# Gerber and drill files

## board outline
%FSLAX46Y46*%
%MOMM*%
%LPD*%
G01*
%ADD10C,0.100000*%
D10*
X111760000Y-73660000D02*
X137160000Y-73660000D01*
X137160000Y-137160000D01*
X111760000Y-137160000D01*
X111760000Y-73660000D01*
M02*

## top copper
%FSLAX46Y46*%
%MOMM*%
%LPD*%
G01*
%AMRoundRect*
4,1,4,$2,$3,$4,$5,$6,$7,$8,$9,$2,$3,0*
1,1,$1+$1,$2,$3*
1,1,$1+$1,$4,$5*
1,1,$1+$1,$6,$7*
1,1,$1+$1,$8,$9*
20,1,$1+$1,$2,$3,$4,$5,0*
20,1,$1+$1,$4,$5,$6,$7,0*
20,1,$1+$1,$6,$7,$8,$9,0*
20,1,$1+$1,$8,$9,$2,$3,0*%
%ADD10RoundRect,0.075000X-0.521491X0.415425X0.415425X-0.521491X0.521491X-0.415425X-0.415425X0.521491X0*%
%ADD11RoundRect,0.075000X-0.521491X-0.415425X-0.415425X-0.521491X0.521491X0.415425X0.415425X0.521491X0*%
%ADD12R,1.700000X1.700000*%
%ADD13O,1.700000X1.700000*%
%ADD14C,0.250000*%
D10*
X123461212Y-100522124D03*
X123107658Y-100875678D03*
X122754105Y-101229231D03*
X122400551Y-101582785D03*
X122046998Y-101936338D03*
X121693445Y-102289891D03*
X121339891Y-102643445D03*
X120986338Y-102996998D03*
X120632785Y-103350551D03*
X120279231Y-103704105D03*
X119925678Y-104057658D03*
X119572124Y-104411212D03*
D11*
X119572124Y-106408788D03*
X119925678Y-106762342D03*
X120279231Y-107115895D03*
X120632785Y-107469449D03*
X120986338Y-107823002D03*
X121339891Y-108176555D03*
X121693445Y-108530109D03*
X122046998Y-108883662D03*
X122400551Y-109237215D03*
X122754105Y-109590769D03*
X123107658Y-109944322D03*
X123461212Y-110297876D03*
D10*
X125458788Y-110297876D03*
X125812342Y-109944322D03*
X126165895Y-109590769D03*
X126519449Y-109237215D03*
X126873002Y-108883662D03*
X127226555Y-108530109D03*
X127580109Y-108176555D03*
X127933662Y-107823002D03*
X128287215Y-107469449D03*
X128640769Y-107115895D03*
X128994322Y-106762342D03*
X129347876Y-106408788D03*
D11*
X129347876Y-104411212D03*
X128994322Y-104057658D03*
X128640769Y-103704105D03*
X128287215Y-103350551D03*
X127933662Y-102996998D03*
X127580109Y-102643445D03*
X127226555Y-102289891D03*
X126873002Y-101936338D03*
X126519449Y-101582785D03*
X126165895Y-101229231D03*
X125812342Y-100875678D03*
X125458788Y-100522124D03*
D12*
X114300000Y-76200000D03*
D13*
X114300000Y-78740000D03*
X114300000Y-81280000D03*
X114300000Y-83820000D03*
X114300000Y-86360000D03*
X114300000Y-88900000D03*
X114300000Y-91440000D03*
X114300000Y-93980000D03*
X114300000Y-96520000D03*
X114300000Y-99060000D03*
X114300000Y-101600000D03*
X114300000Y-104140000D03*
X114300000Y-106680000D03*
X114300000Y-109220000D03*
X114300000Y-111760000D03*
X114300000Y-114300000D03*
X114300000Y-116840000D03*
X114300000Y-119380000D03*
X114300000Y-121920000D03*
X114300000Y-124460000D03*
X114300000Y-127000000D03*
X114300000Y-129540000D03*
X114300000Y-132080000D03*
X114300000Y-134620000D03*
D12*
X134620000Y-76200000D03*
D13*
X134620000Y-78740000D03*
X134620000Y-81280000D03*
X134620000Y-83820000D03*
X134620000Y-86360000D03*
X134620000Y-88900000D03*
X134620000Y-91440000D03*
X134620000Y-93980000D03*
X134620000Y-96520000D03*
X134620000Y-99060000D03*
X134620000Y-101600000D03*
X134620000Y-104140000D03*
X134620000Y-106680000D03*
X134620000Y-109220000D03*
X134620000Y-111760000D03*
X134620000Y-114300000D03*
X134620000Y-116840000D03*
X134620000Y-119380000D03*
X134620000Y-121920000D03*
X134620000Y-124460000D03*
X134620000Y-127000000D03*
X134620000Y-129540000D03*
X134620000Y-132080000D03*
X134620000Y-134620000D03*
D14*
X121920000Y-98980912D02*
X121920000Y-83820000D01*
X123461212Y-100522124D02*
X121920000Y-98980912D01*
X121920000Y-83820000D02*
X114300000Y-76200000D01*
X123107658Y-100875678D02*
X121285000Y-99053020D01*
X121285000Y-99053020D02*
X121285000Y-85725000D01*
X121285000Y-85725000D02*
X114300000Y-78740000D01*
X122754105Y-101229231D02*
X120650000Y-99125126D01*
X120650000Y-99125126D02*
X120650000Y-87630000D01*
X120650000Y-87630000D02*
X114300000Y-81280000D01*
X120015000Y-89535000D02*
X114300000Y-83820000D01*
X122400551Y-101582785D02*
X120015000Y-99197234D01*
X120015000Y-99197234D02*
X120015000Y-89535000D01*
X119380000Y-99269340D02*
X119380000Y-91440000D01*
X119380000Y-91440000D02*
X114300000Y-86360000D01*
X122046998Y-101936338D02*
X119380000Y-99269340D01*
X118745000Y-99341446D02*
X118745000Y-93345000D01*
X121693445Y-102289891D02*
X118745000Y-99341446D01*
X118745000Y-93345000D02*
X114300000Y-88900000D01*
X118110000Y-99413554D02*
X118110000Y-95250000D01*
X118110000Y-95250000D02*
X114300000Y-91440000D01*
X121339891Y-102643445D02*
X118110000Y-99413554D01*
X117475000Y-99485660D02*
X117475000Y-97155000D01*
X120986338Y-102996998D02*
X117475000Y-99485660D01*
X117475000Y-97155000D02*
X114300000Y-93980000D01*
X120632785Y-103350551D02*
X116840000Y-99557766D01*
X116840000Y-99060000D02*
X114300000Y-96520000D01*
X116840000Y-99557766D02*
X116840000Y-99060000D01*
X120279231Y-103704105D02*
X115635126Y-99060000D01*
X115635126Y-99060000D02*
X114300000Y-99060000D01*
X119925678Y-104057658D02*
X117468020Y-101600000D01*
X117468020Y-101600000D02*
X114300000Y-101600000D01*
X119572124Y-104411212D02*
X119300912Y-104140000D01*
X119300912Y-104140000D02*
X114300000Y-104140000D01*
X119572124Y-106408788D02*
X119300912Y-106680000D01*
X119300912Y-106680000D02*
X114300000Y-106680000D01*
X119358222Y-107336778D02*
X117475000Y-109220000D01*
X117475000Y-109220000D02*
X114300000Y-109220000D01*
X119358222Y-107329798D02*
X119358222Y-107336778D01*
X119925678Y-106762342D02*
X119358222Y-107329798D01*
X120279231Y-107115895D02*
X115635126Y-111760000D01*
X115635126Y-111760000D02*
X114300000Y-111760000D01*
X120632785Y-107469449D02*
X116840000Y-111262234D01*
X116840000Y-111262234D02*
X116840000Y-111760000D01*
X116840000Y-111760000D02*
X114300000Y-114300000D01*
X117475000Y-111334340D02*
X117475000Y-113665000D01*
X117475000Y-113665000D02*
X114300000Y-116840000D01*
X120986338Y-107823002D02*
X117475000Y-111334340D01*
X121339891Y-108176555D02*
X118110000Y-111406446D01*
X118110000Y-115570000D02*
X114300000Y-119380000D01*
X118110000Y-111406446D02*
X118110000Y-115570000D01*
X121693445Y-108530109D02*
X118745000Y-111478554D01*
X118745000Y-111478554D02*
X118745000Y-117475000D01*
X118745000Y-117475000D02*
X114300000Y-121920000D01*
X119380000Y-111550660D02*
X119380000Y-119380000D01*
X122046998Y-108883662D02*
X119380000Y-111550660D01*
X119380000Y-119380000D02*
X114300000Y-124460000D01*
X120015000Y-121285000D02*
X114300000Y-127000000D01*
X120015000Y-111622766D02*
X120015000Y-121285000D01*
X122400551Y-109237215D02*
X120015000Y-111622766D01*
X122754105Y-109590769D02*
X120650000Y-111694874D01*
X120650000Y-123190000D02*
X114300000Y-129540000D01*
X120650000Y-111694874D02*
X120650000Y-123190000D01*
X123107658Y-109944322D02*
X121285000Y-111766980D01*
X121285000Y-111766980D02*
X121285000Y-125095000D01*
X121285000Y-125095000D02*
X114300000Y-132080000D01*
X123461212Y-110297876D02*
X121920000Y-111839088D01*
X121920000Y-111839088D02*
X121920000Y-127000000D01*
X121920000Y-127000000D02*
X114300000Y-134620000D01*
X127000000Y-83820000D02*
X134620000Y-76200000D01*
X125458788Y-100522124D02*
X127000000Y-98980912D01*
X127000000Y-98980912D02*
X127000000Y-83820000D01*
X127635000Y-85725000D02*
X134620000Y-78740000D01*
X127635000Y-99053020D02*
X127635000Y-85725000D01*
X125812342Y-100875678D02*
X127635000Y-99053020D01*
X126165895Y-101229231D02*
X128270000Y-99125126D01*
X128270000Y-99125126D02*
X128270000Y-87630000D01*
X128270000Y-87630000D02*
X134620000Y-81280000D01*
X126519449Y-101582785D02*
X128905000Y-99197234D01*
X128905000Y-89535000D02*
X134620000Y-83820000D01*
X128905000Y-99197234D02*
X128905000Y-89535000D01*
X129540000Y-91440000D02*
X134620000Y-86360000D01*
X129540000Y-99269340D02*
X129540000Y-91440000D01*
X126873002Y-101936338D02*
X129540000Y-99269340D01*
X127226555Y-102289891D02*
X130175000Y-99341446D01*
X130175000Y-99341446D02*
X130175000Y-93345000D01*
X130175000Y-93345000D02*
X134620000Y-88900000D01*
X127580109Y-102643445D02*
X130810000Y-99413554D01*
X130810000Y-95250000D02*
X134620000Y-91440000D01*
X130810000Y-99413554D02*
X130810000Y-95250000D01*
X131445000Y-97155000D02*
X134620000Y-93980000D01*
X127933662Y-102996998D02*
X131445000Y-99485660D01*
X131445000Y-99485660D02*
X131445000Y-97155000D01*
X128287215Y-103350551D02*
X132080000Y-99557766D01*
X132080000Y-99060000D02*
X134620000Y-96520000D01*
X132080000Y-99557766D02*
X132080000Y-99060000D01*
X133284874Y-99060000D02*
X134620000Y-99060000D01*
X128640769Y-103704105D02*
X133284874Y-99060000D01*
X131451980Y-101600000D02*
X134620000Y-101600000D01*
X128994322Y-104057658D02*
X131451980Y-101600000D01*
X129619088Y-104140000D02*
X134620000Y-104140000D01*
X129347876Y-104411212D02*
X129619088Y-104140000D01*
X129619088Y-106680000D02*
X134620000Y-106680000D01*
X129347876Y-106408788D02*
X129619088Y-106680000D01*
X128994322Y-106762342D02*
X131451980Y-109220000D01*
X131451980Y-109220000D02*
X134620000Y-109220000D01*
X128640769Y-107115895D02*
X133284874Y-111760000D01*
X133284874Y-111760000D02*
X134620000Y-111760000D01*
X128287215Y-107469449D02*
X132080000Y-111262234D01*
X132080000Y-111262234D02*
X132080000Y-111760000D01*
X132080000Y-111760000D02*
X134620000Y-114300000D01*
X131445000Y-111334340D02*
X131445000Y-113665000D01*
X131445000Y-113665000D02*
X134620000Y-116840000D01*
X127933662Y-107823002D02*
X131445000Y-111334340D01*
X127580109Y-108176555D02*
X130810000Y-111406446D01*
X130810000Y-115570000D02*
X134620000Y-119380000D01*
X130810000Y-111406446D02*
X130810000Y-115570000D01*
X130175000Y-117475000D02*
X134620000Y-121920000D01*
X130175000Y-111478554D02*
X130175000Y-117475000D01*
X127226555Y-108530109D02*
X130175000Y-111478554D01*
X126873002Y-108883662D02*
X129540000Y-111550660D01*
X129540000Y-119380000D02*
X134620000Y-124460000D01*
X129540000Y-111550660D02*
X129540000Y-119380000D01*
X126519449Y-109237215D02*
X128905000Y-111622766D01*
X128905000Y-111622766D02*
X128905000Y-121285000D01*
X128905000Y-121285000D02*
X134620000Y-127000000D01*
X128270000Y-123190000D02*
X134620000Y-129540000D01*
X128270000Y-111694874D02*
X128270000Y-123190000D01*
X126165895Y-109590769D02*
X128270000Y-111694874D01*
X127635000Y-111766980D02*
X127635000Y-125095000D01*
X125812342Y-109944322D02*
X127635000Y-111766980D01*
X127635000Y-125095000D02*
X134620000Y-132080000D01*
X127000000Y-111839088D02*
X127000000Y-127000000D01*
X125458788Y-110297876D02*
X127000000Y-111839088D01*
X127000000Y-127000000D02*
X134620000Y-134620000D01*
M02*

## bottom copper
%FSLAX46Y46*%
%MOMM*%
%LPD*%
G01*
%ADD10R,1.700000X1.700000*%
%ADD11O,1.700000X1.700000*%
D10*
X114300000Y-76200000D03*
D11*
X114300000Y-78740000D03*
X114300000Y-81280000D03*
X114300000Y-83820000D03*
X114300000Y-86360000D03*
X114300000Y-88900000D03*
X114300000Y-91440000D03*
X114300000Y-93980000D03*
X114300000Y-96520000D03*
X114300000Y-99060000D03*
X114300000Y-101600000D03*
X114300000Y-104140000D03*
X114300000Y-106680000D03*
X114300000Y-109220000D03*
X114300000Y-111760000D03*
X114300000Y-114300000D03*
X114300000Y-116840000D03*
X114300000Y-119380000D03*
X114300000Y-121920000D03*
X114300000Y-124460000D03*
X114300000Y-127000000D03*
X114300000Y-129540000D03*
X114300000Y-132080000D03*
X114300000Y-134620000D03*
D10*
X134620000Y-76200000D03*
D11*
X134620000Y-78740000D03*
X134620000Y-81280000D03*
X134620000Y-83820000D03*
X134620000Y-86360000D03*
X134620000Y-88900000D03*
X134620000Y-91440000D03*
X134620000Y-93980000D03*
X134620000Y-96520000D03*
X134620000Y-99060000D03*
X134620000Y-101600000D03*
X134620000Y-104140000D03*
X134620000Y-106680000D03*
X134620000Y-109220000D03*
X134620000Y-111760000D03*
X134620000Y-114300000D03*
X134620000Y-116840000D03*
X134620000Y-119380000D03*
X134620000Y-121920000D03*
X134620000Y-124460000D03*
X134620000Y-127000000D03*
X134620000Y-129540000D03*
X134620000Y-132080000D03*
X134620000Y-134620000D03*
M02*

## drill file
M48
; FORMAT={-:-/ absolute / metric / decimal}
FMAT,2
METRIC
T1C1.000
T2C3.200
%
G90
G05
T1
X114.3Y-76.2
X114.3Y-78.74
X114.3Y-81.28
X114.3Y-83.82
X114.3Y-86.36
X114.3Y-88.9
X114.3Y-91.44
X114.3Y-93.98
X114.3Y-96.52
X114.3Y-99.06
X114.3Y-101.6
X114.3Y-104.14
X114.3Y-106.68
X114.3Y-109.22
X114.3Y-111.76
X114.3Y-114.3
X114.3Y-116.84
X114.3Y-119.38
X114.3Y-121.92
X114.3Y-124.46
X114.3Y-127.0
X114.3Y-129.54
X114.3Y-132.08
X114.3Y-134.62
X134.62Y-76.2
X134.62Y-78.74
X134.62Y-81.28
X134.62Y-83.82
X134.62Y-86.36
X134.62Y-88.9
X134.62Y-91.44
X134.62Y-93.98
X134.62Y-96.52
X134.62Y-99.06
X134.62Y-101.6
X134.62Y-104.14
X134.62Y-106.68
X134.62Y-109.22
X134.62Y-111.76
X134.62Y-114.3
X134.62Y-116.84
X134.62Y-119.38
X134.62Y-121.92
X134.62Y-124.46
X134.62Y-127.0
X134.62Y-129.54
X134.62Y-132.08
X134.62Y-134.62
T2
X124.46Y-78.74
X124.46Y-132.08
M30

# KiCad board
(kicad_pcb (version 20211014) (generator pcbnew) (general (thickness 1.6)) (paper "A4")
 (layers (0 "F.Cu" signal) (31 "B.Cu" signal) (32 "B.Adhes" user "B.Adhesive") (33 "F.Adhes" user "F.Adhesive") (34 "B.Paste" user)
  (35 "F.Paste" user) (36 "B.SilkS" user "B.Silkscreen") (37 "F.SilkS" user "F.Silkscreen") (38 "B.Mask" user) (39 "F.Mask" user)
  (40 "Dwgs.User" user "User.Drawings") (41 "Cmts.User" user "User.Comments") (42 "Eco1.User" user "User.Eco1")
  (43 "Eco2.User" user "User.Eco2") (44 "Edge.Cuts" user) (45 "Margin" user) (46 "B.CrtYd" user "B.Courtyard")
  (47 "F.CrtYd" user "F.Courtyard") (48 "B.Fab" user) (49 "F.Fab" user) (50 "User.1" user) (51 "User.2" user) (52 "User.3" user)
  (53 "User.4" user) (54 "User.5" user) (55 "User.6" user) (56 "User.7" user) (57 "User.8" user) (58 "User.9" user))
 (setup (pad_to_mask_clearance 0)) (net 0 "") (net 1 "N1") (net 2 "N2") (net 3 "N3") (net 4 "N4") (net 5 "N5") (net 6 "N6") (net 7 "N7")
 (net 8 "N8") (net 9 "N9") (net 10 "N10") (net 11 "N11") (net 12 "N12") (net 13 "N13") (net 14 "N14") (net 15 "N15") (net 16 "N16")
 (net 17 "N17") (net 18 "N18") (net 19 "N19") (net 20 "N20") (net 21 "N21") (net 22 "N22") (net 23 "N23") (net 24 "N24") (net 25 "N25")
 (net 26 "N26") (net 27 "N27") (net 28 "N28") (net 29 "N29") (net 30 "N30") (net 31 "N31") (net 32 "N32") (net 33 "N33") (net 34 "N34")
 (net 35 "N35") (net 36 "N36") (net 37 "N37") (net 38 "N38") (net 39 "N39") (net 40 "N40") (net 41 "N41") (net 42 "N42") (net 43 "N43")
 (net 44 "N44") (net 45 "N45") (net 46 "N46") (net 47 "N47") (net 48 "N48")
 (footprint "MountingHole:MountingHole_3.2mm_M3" (layer "F.Cu") (at 124.46 78.74)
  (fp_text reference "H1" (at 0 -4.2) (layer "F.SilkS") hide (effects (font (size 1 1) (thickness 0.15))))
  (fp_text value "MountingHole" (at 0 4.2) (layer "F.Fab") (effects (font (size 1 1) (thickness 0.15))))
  (pad "" np_thru_hole circle (at 0 0) (size 3.2 3.2) (drill 3.2) (layers *.Cu *.Mask)))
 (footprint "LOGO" (layer "F.Cu") (at 124.46 94.615 90)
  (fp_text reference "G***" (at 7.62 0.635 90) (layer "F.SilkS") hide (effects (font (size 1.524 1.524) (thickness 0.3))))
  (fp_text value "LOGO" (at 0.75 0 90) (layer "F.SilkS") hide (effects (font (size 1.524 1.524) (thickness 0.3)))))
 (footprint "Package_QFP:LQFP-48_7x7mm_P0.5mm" (layer "F.Cu") (at 124.46 105.41 -45)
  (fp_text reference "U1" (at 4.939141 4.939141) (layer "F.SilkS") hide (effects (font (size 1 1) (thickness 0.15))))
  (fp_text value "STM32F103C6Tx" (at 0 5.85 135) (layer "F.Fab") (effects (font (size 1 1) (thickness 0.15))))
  (pad "1" smd roundrect (at -4.1625 -2.75 315) (size 1.475 0.3) (layers "F.Cu" "F.Paste" "F.Mask") (roundrect_rratio 0.25) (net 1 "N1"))
  (pad "2" smd roundrect (at -4.1625 -2.25 315) (size 1.475 0.3) (layers "F.Cu" "F.Paste" "F.Mask") (roundrect_rratio 0.25) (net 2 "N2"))
  (pad "3" smd roundrect (at -4.1625 -1.75 315) (size 1.475 0.3) (layers "F.Cu" "F.Paste" "F.Mask") (roundrect_rratio 0.25) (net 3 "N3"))
  (pad "4" smd roundrect (at -4.1625 -1.25 315) (size 1.475 0.3) (layers "F.Cu" "F.Paste" "F.Mask") (roundrect_rratio 0.25) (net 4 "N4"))
  (pad "5" smd roundrect (at -4.1625 -0.75 315) (size 1.475 0.3) (layers "F.Cu" "F.Paste" "F.Mask") (roundrect_rratio 0.25) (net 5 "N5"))
  (pad "6" smd roundrect (at -4.1625 -0.25 315) (size 1.475 0.3) (layers "F.Cu" "F.Paste" "F.Mask") (roundrect_rratio 0.25) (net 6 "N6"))
  (pad "7" smd roundrect (at -4.1625 0.25 315) (size 1.475 0.3) (layers "F.Cu" "F.Paste" "F.Mask") (roundrect_rratio 0.25) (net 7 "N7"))
  (pad "8" smd roundrect (at -4.1625 0.75 315) (size 1.475 0.3) (layers "F.Cu" "F.Paste" "F.Mask") (roundrect_rratio 0.25) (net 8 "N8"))
  (pad "9" smd roundrect (at -4.1625 1.25 315) (size 1.475 0.3) (layers "F.Cu" "F.Paste" "F.Mask") (roundrect_rratio 0.25) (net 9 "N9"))
  (pad "10" smd roundrect (at -4.1625 1.75 315) (size 1.475 0.3) (layers "F.Cu" "F.Paste" "F.Mask") (roundrect_rratio 0.25) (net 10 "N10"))
  (pad "11" smd roundrect (at -4.1625 2.25 315) (size 1.475 0.3) (layers "F.Cu" "F.Paste" "F.Mask") (roundrect_rratio 0.25) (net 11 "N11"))
  (pad "12" smd roundrect (at -4.1625 2.75 315) (size 1.475 0.3) (layers "F.Cu" "F.Paste" "F.Mask") (roundrect_rratio 0.25) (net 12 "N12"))
  (pad "13" smd roundrect (at -2.75 4.1625 315) (size 0.3 1.475) (layers "F.Cu" "F.Paste" "F.Mask") (roundrect_rratio 0.25) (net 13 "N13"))
  (pad "14" smd roundrect (at -2.25 4.1625 315) (size 0.3 1.475) (layers "F.Cu" "F.Paste" "F.Mask") (roundrect_rratio 0.25) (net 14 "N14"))
  (pad "15" smd roundrect (at -1.75 4.1625 315) (size 0.3 1.475) (layers "F.Cu" "F.Paste" "F.Mask") (roundrect_rratio 0.25) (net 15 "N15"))
  (pad "16" smd roundrect (at -1.25 4.1625 315) (size 0.3 1.475) (layers "F.Cu" "F.Paste" "F.Mask") (roundrect_rratio 0.25) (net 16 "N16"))
  (pad "17" smd roundrect (at -0.75 4.1625 315) (size 0.3 1.475) (layers "F.Cu" "F.Paste" "F.Mask") (roundrect_rratio 0.25) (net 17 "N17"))
  (pad "18" smd roundrect (at -0.25 4.1625 315) (size 0.3 1.475) (layers "F.Cu" "F.Paste" "F.Mask") (roundrect_rratio 0.25) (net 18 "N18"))
  (pad "19" smd roundrect (at 0.25 4.1625 315) (size 0.3 1.475) (layers "F.Cu" "F.Paste" "F.Mask") (roundrect_rratio 0.25) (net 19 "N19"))
  (pad "20" smd roundrect (at 0.75 4.1625 315) (size 0.3 1.475) (layers "F.Cu" "F.Paste" "F.Mask") (roundrect_rratio 0.25) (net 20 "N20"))
  (pad "21" smd roundrect (at 1.25 4.1625 315) (size 0.3 1.475) (layers "F.Cu" "F.Paste" "F.Mask") (roundrect_rratio 0.25) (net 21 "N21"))
  (pad "22" smd roundrect (at 1.75 4.1625 315) (size 0.3 1.475) (layers "F.Cu" "F.Paste" "F.Mask") (roundrect_rratio 0.25) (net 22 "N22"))
  (pad "23" smd roundrect (at 2.25 4.1625 315) (size 0.3 1.475) (layers "F.Cu" "F.Paste" "F.Mask") (roundrect_rratio 0.25) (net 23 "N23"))
  (pad "24" smd roundrect (at 2.75 4.1625 315) (size 0.3 1.475) (layers "F.Cu" "F.Paste" "F.Mask") (roundrect_rratio 0.25) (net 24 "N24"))
  (pad "25" smd roundrect (at 4.1625 2.75 315) (size 1.475 0.3) (layers "F.Cu" "F.Paste" "F.Mask") (roundrect_rratio 0.25) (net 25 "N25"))
  (pad "26" smd roundrect (at 4.1625 2.25 315) (size 1.475 0.3) (layers "F.Cu" "F.Paste" "F.Mask") (roundrect_rratio 0.25) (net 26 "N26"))
  (pad "27" smd roundrect (at 4.1625 1.75 315) (size 1.475 0.3) (layers "F.Cu" "F.Paste" "F.Mask") (roundrect_rratio 0.25) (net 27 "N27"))
  (pad "28" smd roundrect (at 4.1625 1.25 315) (size 1.475 0.3) (layers "F.Cu" "F.Paste" "F.Mask") (roundrect_rratio 0.25) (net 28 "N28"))
  (pad "29" smd roundrect (at 4.1625 0.75 315) (size 1.475 0.3) (layers "F.Cu" "F.Paste" "F.Mask") (roundrect_rratio 0.25) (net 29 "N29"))
  (pad "30" smd roundrect (at 4.1625 0.25 315) (size 1.475 0.3) (layers "F.Cu" "F.Paste" "F.Mask") (roundrect_rratio 0.25) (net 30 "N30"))
  (pad "31" smd roundrect (at 4.1625 -0.25 315) (size 1.475 0.3) (layers "F.Cu" "F.Paste" "F.Mask") (roundrect_rratio 0.25) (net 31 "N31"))
  (pad "32" smd roundrect (at 4.1625 -0.75 315) (size 1.475 0.3) (layers "F.Cu" "F.Paste" "F.Mask") (roundrect_rratio 0.25) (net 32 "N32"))
  (pad "33" smd roundrect (at 4.1625 -1.25 315) (size 1.475 0.3) (layers "F.Cu" "F.Paste" "F.Mask") (roundrect_rratio 0.25) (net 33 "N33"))
  (pad "34" smd roundrect (at 4.1625 -1.75 315) (size 1.475 0.3) (layers "F.Cu" "F.Paste" "F.Mask") (roundrect_rratio 0.25) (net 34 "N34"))
  (pad "35" smd roundrect (at 4.1625 -2.25 315) (size 1.475 0.3) (layers "F.Cu" "F.Paste" "F.Mask") (roundrect_rratio 0.25) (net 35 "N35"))
  (pad "36" smd roundrect (at 4.1625 -2.75 315) (size 1.475 0.3) (layers "F.Cu" "F.Paste" "F.Mask") (roundrect_rratio 0.25) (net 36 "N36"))
  (pad "37" smd roundrect (at 2.75 -4.1625 315) (size 0.3 1.475) (layers "F.Cu" "F.Paste" "F.Mask") (roundrect_rratio 0.25) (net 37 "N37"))
  (pad "38" smd roundrect (at 2.25 -4.1625 315) (size 0.3 1.475) (layers "F.Cu" "F.Paste" "F.Mask") (roundrect_rratio 0.25) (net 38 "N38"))
  (pad "39" smd roundrect (at 1.75 -4.1625 315) (size 0.3 1.475) (layers "F.Cu" "F.Paste" "F.Mask") (roundrect_rratio 0.25) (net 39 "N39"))
  (pad "40" smd roundrect (at 1.25 -4.1625 315) (size 0.3 1.475) (layers "F.Cu" "F.Paste" "F.Mask") (roundrect_rratio 0.25) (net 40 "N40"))
  (pad "41" smd roundrect (at 0.75 -4.1625 315) (size 0.3 1.475) (layers "F.Cu" "F.Paste" "F.Mask") (roundrect_rratio 0.25) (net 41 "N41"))
  (pad "42" smd roundrect (at 0.25 -4.1625 315) (size 0.3 1.475) (layers "F.Cu" "F.Paste" "F.Mask") (roundrect_rratio 0.25) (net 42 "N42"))
  (pad "43" smd roundrect (at -0.25 -4.1625 315) (size 0.3 1.475) (layers "F.Cu" "F.Paste" "F.Mask") (roundrect_rratio 0.25) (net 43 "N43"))
  (pad "44" smd roundrect (at -0.75 -4.1625 315) (size 0.3 1.475) (layers "F.Cu" "F.Paste" "F.Mask") (roundrect_rratio 0.25) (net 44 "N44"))
  (pad "45" smd roundrect (at -1.25 -4.1625 315) (size 0.3 1.475) (layers "F.Cu" "F.Paste" "F.Mask") (roundrect_rratio 0.25) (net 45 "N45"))
  (pad "46" smd roundrect (at -1.75 -4.1625 315) (size 0.3 1.475) (layers "F.Cu" "F.Paste" "F.Mask") (roundrect_rratio 0.25) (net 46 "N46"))
  (pad "47" smd roundrect (at -2.25 -4.1625 315) (size 0.3 1.475) (layers "F.Cu" "F.Paste" "F.Mask") (roundrect_rratio 0.25) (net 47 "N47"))
  (pad "48" smd roundrect (at -2.75 -4.1625 315) (size 0.3 1.475) (layers "F.Cu" "F.Paste" "F.Mask") (roundrect_rratio 0.25) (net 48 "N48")))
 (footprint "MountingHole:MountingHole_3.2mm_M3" (layer "F.Cu") (at 124.46 132.08)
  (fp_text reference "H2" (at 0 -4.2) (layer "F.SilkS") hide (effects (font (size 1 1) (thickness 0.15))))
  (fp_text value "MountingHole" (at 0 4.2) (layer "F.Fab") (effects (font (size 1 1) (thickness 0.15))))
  (pad "" np_thru_hole circle (at 0 0) (size 3.2 3.2) (drill 3.2) (layers *.Cu *.Mask)))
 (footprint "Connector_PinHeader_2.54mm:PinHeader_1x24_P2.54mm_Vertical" (layer "B.Cu") (at 114.3 76.2 180)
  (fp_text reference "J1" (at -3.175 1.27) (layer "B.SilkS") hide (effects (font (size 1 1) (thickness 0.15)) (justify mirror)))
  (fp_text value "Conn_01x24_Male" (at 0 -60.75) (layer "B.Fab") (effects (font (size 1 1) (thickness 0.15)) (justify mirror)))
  (pad "1" thru_hole rect (at 0 0 180) (size 1.7 1.7) (drill 1) (layers *.Cu *.Mask) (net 1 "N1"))
  (pad "2" thru_hole oval (at 0 -2.54 180) (size 1.7 1.7) (drill 1) (layers *.Cu *.Mask) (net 2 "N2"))
  (pad "3" thru_hole oval (at 0 -5.08 180) (size 1.7 1.7) (drill 1) (layers *.Cu *.Mask) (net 3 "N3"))
  (pad "4" thru_hole oval (at 0 -7.62 180) (size 1.7 1.7) (drill 1) (layers *.Cu *.Mask) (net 4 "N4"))
  (pad "5" thru_hole oval (at 0 -10.16 180) (size 1.7 1.7) (drill 1) (layers *.Cu *.Mask) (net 5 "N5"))
  (pad "6" thru_hole oval (at 0 -12.7 180) (size 1.7 1.7) (drill 1) (layers *.Cu *.Mask) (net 6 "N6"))
  (pad "7" thru_hole oval (at 0 -15.24 180) (size 1.7 1.7) (drill 1) (layers *.Cu *.Mask) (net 7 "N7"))
  (pad "8" thru_hole oval (at 0 -17.78 180) (size 1.7 1.7) (drill 1) (layers *.Cu *.Mask) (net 8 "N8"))
  (pad "9" thru_hole oval (at 0 -20.32 180) (size 1.7 1.7) (drill 1) (layers *.Cu *.Mask) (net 9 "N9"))
  (pad "10" thru_hole oval (at 0 -22.86 180) (size 1.7 1.7) (drill 1) (layers *.Cu *.Mask) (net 10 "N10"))
  (pad "11" thru_hole oval (at 0 -25.4 180) (size 1.7 1.7) (drill 1) (layers *.Cu *.Mask) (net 11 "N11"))
  (pad "12" thru_hole oval (at 0 -27.94 180) (size 1.7 1.7) (drill 1) (layers *.Cu *.Mask) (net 12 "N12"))
  (pad "13" thru_hole oval (at 0 -30.48 180) (size 1.7 1.7) (drill 1) (layers *.Cu *.Mask) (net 13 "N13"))
  (pad "14" thru_hole oval (at 0 -33.02 180) (size 1.7 1.7) (drill 1) (layers *.Cu *.Mask) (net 14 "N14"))
  (pad "15" thru_hole oval (at 0 -35.56 180) (size 1.7 1.7) (drill 1) (layers *.Cu *.Mask) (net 15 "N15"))
  (pad "16" thru_hole oval (at 0 -38.1 180) (size 1.7 1.7) (drill 1) (layers *.Cu *.Mask) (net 16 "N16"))
  (pad "17" thru_hole oval (at 0 -40.64 180) (size 1.7 1.7) (drill 1) (layers *.Cu *.Mask) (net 17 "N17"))
  (pad "18" thru_hole oval (at 0 -43.18 180) (size 1.7 1.7) (drill 1) (layers *.Cu *.Mask) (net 18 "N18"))
  (pad "19" thru_hole oval (at 0 -45.72 180) (size 1.7 1.7) (drill 1) (layers *.Cu *.Mask) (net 19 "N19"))
  (pad "20" thru_hole oval (at 0 -48.26 180) (size 1.7 1.7) (drill 1) (layers *.Cu *.Mask) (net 20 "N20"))
  (pad "21" thru_hole oval (at 0 -50.8 180) (size 1.7 1.7) (drill 1) (layers *.Cu *.Mask) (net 21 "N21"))
  (pad "22" thru_hole oval (at 0 -53.34 180) (size 1.7 1.7) (drill 1) (layers *.Cu *.Mask) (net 22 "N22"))
  (pad "23" thru_hole oval (at 0 -55.88 180) (size 1.7 1.7) (drill 1) (layers *.Cu *.Mask) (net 23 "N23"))
  (pad "24" thru_hole oval (at 0 -58.42 180) (size 1.7 1.7) (drill 1) (layers *.Cu *.Mask) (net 24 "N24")))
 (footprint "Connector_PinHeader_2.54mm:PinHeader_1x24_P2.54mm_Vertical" (layer "B.Cu") (at 134.62 76.2 180)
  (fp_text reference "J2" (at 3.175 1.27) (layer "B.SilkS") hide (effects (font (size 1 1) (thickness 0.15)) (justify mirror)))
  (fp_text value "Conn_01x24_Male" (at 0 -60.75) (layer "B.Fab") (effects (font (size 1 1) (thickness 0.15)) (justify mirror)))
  (pad "1" thru_hole rect (at 0 0 180) (size 1.7 1.7) (drill 1) (layers *.Cu *.Mask) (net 48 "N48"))
  (pad "2" thru_hole oval (at 0 -2.54 180) (size 1.7 1.7) (drill 1) (layers *.Cu *.Mask) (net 47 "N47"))
  (pad "3" thru_hole oval (at 0 -5.08 180) (size 1.7 1.7) (drill 1) (layers *.Cu *.Mask) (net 46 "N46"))
  (pad "4" thru_hole oval (at 0 -7.62 180) (size 1.7 1.7) (drill 1) (layers *.Cu *.Mask) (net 45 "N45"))
  (pad "5" thru_hole oval (at 0 -10.16 180) (size 1.7 1.7) (drill 1) (layers *.Cu *.Mask) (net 44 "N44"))
  (pad "6" thru_hole oval (at 0 -12.7 180) (size 1.7 1.7) (drill 1) (layers *.Cu *.Mask) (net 43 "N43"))
  (pad "7" thru_hole oval (at 0 -15.24 180) (size 1.7 1.7) (drill 1) (layers *.Cu *.Mask) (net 42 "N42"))
  (pad "8" thru_hole oval (at 0 -17.78 180) (size 1.7 1.7) (drill 1) (layers *.Cu *.Mask) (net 41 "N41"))
  (pad "9" thru_hole oval (at 0 -20.32 180) (size 1.7 1.7) (drill 1) (layers *.Cu *.Mask) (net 40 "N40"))
  (pad "10" thru_hole oval (at 0 -22.86 180) (size 1.7 1.7) (drill 1) (layers *.Cu *.Mask) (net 39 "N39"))
  (pad "11" thru_hole oval (at 0 -25.4 180) (size 1.7 1.7) (drill 1) (layers *.Cu *.Mask) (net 38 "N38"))
  (pad "12" thru_hole oval (at 0 -27.94 180) (size 1.7 1.7) (drill 1) (layers *.Cu *.Mask) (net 37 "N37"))
  (pad "13" thru_hole oval (at 0 -30.48 180) (size 1.7 1.7) (drill 1) (layers *.Cu *.Mask) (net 36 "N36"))
  (pad "14" thru_hole oval (at 0 -33.02 180) (size 1.7 1.7) (drill 1) (layers *.Cu *.Mask) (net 35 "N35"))
  (pad "15" thru_hole oval (at 0 -35.56 180) (size 1.7 1.7) (drill 1) (layers *.Cu *.Mask) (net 34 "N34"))
  (pad "16" thru_hole oval (at 0 -38.1 180) (size 1.7 1.7) (drill 1) (layers *.Cu *.Mask) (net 33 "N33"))
  (pad "17" thru_hole oval (at 0 -40.64 180) (size 1.7 1.7) (drill 1) (layers *.Cu *.Mask) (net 32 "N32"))
  (pad "18" thru_hole oval (at 0 -43.18 180) (size 1.7 1.7) (drill 1) (layers *.Cu *.Mask) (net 31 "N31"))
  (pad "19" thru_hole oval (at 0 -45.72 180) (size 1.7 1.7) (drill 1) (layers *.Cu *.Mask) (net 30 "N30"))
  (pad "20" thru_hole oval (at 0 -48.26 180) (size 1.7 1.7) (drill 1) (layers *.Cu *.Mask) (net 29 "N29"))
  (pad "21" thru_hole oval (at 0 -50.8 180) (size 1.7 1.7) (drill 1) (layers *.Cu *.Mask) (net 28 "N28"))
  (pad "22" thru_hole oval (at 0 -53.34 180) (size 1.7 1.7) (drill 1) (layers *.Cu *.Mask) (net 27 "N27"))
  (pad "23" thru_hole oval (at 0 -55.88 180) (size 1.7 1.7) (drill 1) (layers *.Cu *.Mask) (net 26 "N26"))
  (pad "24" thru_hole oval (at 0 -58.42 180) (size 1.7 1.7) (drill 1) (layers *.Cu *.Mask) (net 25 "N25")))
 (gr_rect (start 111.76 73.66) (end 137.16 137.16) (layer "Edge.Cuts") (width 0.1) (fill none))
 (segment (start 121.92 98.980912) (end 121.92 83.82) (width 0.25) (layer "F.Cu") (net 1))
 (segment (start 123.461212 100.522124) (end 121.92 98.980912) (width 0.25) (layer "F.Cu") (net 1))
 (segment (start 121.92 83.82) (end 114.3 76.2) (width 0.25) (layer "F.Cu") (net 1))
 (segment (start 123.107658 100.875678) (end 121.285 99.05302) (width 0.25) (layer "F.Cu") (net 2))
 (segment (start 121.285 99.05302) (end 121.285 85.725) (width 0.25) (layer "F.Cu") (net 2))
 (segment (start 121.285 85.725) (end 114.3 78.74) (width 0.25) (layer "F.Cu") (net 2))
 (segment (start 122.754105 101.229231) (end 120.65 99.125126) (width 0.25) (layer "F.Cu") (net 3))
 (segment (start 120.65 99.125126) (end 120.65 87.63) (width 0.25) (layer "F.Cu") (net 3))
 (segment (start 120.65 87.63) (end 114.3 81.28) (width 0.25) (layer "F.Cu") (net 3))
 (segment (start 120.015 89.535) (end 114.3 83.82) (width 0.25) (layer "F.Cu") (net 4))
 (segment (start 122.400551 101.582785) (end 120.015 99.197234) (width 0.25) (layer "F.Cu") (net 4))
 (segment (start 120.015 99.197234) (end 120.015 89.535) (width 0.25) (layer "F.Cu") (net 4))
 (segment (start 119.38 99.26934) (end 119.38 91.44) (width 0.25) (layer "F.Cu") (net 5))
 (segment (start 119.38 91.44) (end 114.3 86.36) (width 0.25) (layer "F.Cu") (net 5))
 (segment (start 122.046998 101.936338) (end 119.38 99.26934) (width 0.25) (layer "F.Cu") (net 5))
 (segment (start 118.745 99.341446) (end 118.745 93.345) (width 0.25) (layer "F.Cu") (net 6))
 (segment (start 121.693445 102.289891) (end 118.745 99.341446) (width 0.25) (layer "F.Cu") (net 6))
 (segment (start 118.745 93.345) (end 114.3 88.9) (width 0.25) (layer "F.Cu") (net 6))
 (segment (start 118.11 99.413554) (end 118.11 95.25) (width 0.25) (layer "F.Cu") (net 7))
 (segment (start 118.11 95.25) (end 114.3 91.44) (width 0.25) (layer "F.Cu") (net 7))
 (segment (start 121.339891 102.643445) (end 118.11 99.413554) (width 0.25) (layer "F.Cu") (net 7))
 (segment (start 117.475 99.48566) (end 117.475 97.155) (width 0.25) (layer "F.Cu") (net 8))
 (segment (start 120.986338 102.996998) (end 117.475 99.48566) (width 0.25) (layer "F.Cu") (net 8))
 (segment (start 117.475 97.155) (end 114.3 93.98) (width 0.25) (layer "F.Cu") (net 8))
 (segment (start 120.632785 103.350551) (end 116.84 99.557766) (width 0.25) (layer "F.Cu") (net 9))
 (segment (start 116.84 99.06) (end 114.3 96.52) (width 0.25) (layer "F.Cu") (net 9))
 (segment (start 116.84 99.557766) (end 116.84 99.06) (width 0.25) (layer "F.Cu") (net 9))
 (segment (start 120.279231 103.704105) (end 115.635126 99.06) (width 0.25) (layer "F.Cu") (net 10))
 (segment (start 115.635126 99.06) (end 114.3 99.06) (width 0.25) (layer "F.Cu") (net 10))
 (segment (start 119.925678 104.057658) (end 117.46802 101.6) (width 0.25) (layer "F.Cu") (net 11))
 (segment (start 117.46802 101.6) (end 114.3 101.6) (width 0.25) (layer "F.Cu") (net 11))
 (segment (start 119.572124 104.411212) (end 119.300912 104.14) (width 0.25) (layer "F.Cu") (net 12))
 (segment (start 119.300912 104.14) (end 114.3 104.14) (width 0.25) (layer "F.Cu") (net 12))
 (segment (start 119.572124 106.408788) (end 119.300912 106.68) (width 0.25) (layer "F.Cu") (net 13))
 (segment (start 119.300912 106.68) (end 114.3 106.68) (width 0.25) (layer "F.Cu") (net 13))
 (segment (start 119.358222 107.336778) (end 117.475 109.22) (width 0.25) (layer "F.Cu") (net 14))
 (segment (start 117.475 109.22) (end 114.3 109.22) (width 0.25) (layer "F.Cu") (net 14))
 (segment (start 119.358222 107.329798) (end 119.358222 107.336778) (width 0.25) (layer "F.Cu") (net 14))
 (segment (start 119.925678 106.762342) (end 119.358222 107.329798) (width 0.25) (layer "F.Cu") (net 14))
 (segment (start 120.279231 107.115895) (end 115.635126 111.76) (width 0.25) (layer "F.Cu") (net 15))
 (segment (start 115.635126 111.76) (end 114.3 111.76) (width 0.25) (layer "F.Cu") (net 15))
 (segment (start 120.632785 107.469449) (end 116.84 111.262234) (width 0.25) (layer "F.Cu") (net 16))
 (segment (start 116.84 111.262234) (end 116.84 111.76) (width 0.25) (layer "F.Cu") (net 16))
 (segment (start 116.84 111.76) (end 114.3 114.3) (width 0.25) (layer "F.Cu") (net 16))
 (segment (start 117.475 111.33434) (end 117.475 113.665) (width 0.25) (layer "F.Cu") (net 17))
 (segment (start 117.475 113.665) (end 114.3 116.84) (width 0.25) (layer "F.Cu") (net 17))
 (segment (start 120.986338 107.823002) (end 117.475 111.33434) (width 0.25) (layer "F.Cu") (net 17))
 (segment (start 121.339891 108.176555) (end 118.11 111.406446) (width 0.25) (layer "F.Cu") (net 18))
 (segment (start 118.11 115.57) (end 114.3 119.38) (width 0.25) (layer "F.Cu") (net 18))
 (segment (start 118.11 111.406446) (end 118.11 115.57) (width 0.25) (layer "F.Cu") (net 18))
 (segment (start 121.693445 108.530109) (end 118.745 111.478554) (width 0.25) (layer "F.Cu") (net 19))
 (segment (start 118.745 111.478554) (end 118.745 117.475) (width 0.25) (layer "F.Cu") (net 19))
 (segment (start 118.745 117.475) (end 114.3 121.92) (width 0.25) (layer "F.Cu") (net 19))
 (segment (start 119.38 111.55066) (end 119.38 119.38) (width 0.25) (layer "F.Cu") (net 20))
 (segment (start 122.046998 108.883662) (end 119.38 111.55066) (width 0.25) (layer "F.Cu") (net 20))
 (segment (start 119.38 119.38) (end 114.3 124.46) (width 0.25) (layer "F.Cu") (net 20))
 (segment (start 120.015 121.285) (end 114.3 127) (width 0.25) (layer "F.Cu") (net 21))
 (segment (start 120.015 111.622766) (end 120.015 121.285) (width 0.25) (layer "F.Cu") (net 21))
 (segment (start 122.400551 109.237215) (end 120.015 111.622766) (width 0.25) (layer "F.Cu") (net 21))
 (segment (start 122.754105 109.590769) (end 120.65 111.694874) (width 0.25) (layer "F.Cu") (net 22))
 (segment (start 120.65 123.19) (end 114.3 129.54) (width 0.25) (layer "F.Cu") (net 22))
 (segment (start 120.65 111.694874) (end 120.65 123.19) (width 0.25) (layer "F.Cu") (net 22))
 (segment (start 123.107658 109.944322) (end 121.285 111.76698) (width 0.25) (layer "F.Cu") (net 23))
 (segment (start 121.285 111.76698) (end 121.285 125.095) (width 0.25) (layer "F.Cu") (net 23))
 (segment (start 121.285 125.095) (end 114.3 132.08) (width 0.25) (layer "F.Cu") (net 23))
 (segment (start 123.461212 110.297876) (end 121.92 111.839088) (width 0.25) (layer "F.Cu") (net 24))
 (segment (start 121.92 111.839088) (end 121.92 127) (width 0.25) (layer "F.Cu") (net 24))
 (segment (start 121.92 127) (end 114.3 134.62) (width 0.25) (layer "F.Cu") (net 24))
 (segment (start 127 83.82) (end 134.62 76.2) (width 0.25) (layer "F.Cu") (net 48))
 (segment (start 125.458788 100.522124) (end 127 98.980912) (width 0.25) (layer "F.Cu") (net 48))
 (segment (start 127 98.980912) (end 127 83.82) (width 0.25) (layer "F.Cu") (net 48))
 (segment (start 127.635 85.725) (end 134.62 78.74) (width 0.25) (layer "F.Cu") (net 47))
 (segment (start 127.635 99.05302) (end 127.635 85.725) (width 0.25) (layer "F.Cu") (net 47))
 (segment (start 125.812342 100.875678) (end 127.635 99.05302) (width 0.25) (layer "F.Cu") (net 47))
 (segment (start 126.165895 101.229231) (end 128.27 99.125126) (width 0.25) (layer "F.Cu") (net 46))
 (segment (start 128.27 99.125126) (end 128.27 87.63) (width 0.25) (layer "F.Cu") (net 46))
 (segment (start 128.27 87.63) (end 134.62 81.28) (width 0.25) (layer "F.Cu") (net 46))
 (segment (start 126.519449 101.582785) (end 128.905 99.197234) (width 0.25) (layer "F.Cu") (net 45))
 (segment (start 128.905 89.535) (end 134.62 83.82) (width 0.25) (layer "F.Cu") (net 45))
 (segment (start 128.905 99.197234) (end 128.905 89.535) (width 0.25) (layer "F.Cu") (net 45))
 (segment (start 129.54 91.44) (end 134.62 86.36) (width 0.25) (layer "F.Cu") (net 44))
 (segment (start 129.54 99.26934) (end 129.54 91.44) (width 0.25) (layer "F.Cu") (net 44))
 (segment (start 126.873002 101.936338) (end 129.54 99.26934) (width 0.25) (layer "F.Cu") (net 44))
 (segment (start 127.226555 102.289891) (end 130.175 99.341446) (width 0.25) (layer "F.Cu") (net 43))
 (segment (start 130.175 99.341446) (end 130.175 93.345) (width 0.25) (layer "F.Cu") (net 43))
 (segment (start 130.175 93.345) (end 134.62 88.9) (width 0.25) (layer "F.Cu") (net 43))
 (segment (start 127.580109 102.643445) (end 130.81 99.413554) (width 0.25) (layer "F.Cu") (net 42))
 (segment (start 130.81 95.25) (end 134.62 91.44) (width 0.25) (layer "F.Cu") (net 42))
 (segment (start 130.81 99.413554) (end 130.81 95.25) (width 0.25) (layer "F.Cu") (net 42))
 (segment (start 131.445 97.155) (end 134.62 93.98) (width 0.25) (layer "F.Cu") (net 41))
 (segment (start 127.933662 102.996998) (end 131.445 99.48566) (width 0.25) (layer "F.Cu") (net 41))
 (segment (start 131.445 99.48566) (end 131.445 97.155) (width 0.25) (layer "F.Cu") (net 41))
 (segment (start 128.287215 103.350551) (end 132.08 99.557766) (width 0.25) (layer "F.Cu") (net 40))
 (segment (start 132.08 99.06) (end 134.62 96.52) (width 0.25) (layer "F.Cu") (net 40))
 (segment (start 132.08 99.557766) (end 132.08 99.06) (width 0.25) (layer "F.Cu") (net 40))
 (segment (start 133.284874 99.06) (end 134.62 99.06) (width 0.25) (layer "F.Cu") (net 39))
 (segment (start 128.640769 103.704105) (end 133.284874 99.06) (width 0.25) (layer "F.Cu") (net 39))
 (segment (start 131.45198 101.6) (end 134.62 101.6) (width 0.25) (layer "F.Cu") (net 38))
 (segment (start 128.994322 104.057658) (end 131.45198 101.6) (width 0.25) (layer "F.Cu") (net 38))
 (segment (start 129.619088 104.14) (end 134.62 104.14) (width 0.25) (layer "F.Cu") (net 37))
 (segment (start 129.347876 104.411212) (end 129.619088 104.14) (width 0.25) (layer "F.Cu") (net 37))
 (segment (start 129.619088 106.68) (end 134.62 106.68) (width 0.25) (layer "F.Cu") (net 36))
 (segment (start 129.347876 106.408788) (end 129.619088 106.68) (width 0.25) (layer "F.Cu") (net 36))
 (segment (start 128.994322 106.762342) (end 131.45198 109.22) (width 0.25) (layer "F.Cu") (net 35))
 (segment (start 131.45198 109.22) (end 134.62 109.22) (width 0.25) (layer "F.Cu") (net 35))
 (segment (start 128.640769 107.115895) (end 133.284874 111.76) (width 0.25) (layer "F.Cu") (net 34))
 (segment (start 133.284874 111.76) (end 134.62 111.76) (width 0.25) (layer "F.Cu") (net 34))
 (segment (start 128.287215 107.469449) (end 132.08 111.262234) (width 0.25) (layer "F.Cu") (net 33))
 (segment (start 132.08 111.262234) (end 132.08 111.76) (width 0.25) (layer "F.Cu") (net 33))
 (segment (start 132.08 111.76) (end 134.62 114.3) (width 0.25) (layer "F.Cu") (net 33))
 (segment (start 131.445 111.33434) (end 131.445 113.665) (width 0.25) (layer "F.Cu") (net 32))
 (segment (start 131.445 113.665) (end 134.62 116.84) (width 0.25) (layer "F.Cu") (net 32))
 (segment (start 127.933662 107.823002) (end 131.445 111.33434) (width 0.25) (layer "F.Cu") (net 32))
 (segment (start 127.580109 108.176555) (end 130.81 111.406446) (width 0.25) (layer "F.Cu") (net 31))
 (segment (start 130.81 115.57) (end 134.62 119.38) (width 0.25) (layer "F.Cu") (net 31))
 (segment (start 130.81 111.406446) (end 130.81 115.57) (width 0.25) (layer "F.Cu") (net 31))
 (segment (start 130.175 117.475) (end 134.62 121.92) (width 0.25) (layer "F.Cu") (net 30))
 (segment (start 130.175 111.478554) (end 130.175 117.475) (width 0.25) (layer "F.Cu") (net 30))
 (segment (start 127.226555 108.530109) (end 130.175 111.478554) (width 0.25) (layer "F.Cu") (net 30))
 (segment (start 126.873002 108.883662) (end 129.54 111.55066) (width 0.25) (layer "F.Cu") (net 29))
 (segment (start 129.54 119.38) (end 134.62 124.46) (width 0.25) (layer "F.Cu") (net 29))
 (segment (start 129.54 111.55066) (end 129.54 119.38) (width 0.25) (layer "F.Cu") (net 29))
 (segment (start 126.519449 109.237215) (end 128.905 111.622766) (width 0.25) (layer "F.Cu") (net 28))
 (segment (start 128.905 111.622766) (end 128.905 121.285) (width 0.25) (layer "F.Cu") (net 28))
 (segment (start 128.905 121.285) (end 134.62 127) (width 0.25) (layer "F.Cu") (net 28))
 (segment (start 128.27 123.19) (end 134.62 129.54) (width 0.25) (layer "F.Cu") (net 27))
 (segment (start 128.27 111.694874) (end 128.27 123.19) (width 0.25) (layer "F.Cu") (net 27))
 (segment (start 126.165895 109.590769) (end 128.27 111.694874) (width 0.25) (layer "F.Cu") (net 27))
 (segment (start 127.635 111.76698) (end 127.635 125.095) (width 0.25) (layer "F.Cu") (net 26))
 (segment (start 125.812342 109.944322) (end 127.635 111.76698) (width 0.25) (layer "F.Cu") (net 26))
 (segment (start 127.635 125.095) (end 134.62 132.08) (width 0.25) (layer "F.Cu") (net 26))
 (segment (start 127 111.839088) (end 127 127) (width 0.25) (layer "F.Cu") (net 25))
 (segment (start 125.458788 110.297876) (end 127 111.839088) (width 0.25) (layer "F.Cu") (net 25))
 (segment (start 127 127) (end 134.62 134.62) (width 0.25) (layer "F.Cu") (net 25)))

